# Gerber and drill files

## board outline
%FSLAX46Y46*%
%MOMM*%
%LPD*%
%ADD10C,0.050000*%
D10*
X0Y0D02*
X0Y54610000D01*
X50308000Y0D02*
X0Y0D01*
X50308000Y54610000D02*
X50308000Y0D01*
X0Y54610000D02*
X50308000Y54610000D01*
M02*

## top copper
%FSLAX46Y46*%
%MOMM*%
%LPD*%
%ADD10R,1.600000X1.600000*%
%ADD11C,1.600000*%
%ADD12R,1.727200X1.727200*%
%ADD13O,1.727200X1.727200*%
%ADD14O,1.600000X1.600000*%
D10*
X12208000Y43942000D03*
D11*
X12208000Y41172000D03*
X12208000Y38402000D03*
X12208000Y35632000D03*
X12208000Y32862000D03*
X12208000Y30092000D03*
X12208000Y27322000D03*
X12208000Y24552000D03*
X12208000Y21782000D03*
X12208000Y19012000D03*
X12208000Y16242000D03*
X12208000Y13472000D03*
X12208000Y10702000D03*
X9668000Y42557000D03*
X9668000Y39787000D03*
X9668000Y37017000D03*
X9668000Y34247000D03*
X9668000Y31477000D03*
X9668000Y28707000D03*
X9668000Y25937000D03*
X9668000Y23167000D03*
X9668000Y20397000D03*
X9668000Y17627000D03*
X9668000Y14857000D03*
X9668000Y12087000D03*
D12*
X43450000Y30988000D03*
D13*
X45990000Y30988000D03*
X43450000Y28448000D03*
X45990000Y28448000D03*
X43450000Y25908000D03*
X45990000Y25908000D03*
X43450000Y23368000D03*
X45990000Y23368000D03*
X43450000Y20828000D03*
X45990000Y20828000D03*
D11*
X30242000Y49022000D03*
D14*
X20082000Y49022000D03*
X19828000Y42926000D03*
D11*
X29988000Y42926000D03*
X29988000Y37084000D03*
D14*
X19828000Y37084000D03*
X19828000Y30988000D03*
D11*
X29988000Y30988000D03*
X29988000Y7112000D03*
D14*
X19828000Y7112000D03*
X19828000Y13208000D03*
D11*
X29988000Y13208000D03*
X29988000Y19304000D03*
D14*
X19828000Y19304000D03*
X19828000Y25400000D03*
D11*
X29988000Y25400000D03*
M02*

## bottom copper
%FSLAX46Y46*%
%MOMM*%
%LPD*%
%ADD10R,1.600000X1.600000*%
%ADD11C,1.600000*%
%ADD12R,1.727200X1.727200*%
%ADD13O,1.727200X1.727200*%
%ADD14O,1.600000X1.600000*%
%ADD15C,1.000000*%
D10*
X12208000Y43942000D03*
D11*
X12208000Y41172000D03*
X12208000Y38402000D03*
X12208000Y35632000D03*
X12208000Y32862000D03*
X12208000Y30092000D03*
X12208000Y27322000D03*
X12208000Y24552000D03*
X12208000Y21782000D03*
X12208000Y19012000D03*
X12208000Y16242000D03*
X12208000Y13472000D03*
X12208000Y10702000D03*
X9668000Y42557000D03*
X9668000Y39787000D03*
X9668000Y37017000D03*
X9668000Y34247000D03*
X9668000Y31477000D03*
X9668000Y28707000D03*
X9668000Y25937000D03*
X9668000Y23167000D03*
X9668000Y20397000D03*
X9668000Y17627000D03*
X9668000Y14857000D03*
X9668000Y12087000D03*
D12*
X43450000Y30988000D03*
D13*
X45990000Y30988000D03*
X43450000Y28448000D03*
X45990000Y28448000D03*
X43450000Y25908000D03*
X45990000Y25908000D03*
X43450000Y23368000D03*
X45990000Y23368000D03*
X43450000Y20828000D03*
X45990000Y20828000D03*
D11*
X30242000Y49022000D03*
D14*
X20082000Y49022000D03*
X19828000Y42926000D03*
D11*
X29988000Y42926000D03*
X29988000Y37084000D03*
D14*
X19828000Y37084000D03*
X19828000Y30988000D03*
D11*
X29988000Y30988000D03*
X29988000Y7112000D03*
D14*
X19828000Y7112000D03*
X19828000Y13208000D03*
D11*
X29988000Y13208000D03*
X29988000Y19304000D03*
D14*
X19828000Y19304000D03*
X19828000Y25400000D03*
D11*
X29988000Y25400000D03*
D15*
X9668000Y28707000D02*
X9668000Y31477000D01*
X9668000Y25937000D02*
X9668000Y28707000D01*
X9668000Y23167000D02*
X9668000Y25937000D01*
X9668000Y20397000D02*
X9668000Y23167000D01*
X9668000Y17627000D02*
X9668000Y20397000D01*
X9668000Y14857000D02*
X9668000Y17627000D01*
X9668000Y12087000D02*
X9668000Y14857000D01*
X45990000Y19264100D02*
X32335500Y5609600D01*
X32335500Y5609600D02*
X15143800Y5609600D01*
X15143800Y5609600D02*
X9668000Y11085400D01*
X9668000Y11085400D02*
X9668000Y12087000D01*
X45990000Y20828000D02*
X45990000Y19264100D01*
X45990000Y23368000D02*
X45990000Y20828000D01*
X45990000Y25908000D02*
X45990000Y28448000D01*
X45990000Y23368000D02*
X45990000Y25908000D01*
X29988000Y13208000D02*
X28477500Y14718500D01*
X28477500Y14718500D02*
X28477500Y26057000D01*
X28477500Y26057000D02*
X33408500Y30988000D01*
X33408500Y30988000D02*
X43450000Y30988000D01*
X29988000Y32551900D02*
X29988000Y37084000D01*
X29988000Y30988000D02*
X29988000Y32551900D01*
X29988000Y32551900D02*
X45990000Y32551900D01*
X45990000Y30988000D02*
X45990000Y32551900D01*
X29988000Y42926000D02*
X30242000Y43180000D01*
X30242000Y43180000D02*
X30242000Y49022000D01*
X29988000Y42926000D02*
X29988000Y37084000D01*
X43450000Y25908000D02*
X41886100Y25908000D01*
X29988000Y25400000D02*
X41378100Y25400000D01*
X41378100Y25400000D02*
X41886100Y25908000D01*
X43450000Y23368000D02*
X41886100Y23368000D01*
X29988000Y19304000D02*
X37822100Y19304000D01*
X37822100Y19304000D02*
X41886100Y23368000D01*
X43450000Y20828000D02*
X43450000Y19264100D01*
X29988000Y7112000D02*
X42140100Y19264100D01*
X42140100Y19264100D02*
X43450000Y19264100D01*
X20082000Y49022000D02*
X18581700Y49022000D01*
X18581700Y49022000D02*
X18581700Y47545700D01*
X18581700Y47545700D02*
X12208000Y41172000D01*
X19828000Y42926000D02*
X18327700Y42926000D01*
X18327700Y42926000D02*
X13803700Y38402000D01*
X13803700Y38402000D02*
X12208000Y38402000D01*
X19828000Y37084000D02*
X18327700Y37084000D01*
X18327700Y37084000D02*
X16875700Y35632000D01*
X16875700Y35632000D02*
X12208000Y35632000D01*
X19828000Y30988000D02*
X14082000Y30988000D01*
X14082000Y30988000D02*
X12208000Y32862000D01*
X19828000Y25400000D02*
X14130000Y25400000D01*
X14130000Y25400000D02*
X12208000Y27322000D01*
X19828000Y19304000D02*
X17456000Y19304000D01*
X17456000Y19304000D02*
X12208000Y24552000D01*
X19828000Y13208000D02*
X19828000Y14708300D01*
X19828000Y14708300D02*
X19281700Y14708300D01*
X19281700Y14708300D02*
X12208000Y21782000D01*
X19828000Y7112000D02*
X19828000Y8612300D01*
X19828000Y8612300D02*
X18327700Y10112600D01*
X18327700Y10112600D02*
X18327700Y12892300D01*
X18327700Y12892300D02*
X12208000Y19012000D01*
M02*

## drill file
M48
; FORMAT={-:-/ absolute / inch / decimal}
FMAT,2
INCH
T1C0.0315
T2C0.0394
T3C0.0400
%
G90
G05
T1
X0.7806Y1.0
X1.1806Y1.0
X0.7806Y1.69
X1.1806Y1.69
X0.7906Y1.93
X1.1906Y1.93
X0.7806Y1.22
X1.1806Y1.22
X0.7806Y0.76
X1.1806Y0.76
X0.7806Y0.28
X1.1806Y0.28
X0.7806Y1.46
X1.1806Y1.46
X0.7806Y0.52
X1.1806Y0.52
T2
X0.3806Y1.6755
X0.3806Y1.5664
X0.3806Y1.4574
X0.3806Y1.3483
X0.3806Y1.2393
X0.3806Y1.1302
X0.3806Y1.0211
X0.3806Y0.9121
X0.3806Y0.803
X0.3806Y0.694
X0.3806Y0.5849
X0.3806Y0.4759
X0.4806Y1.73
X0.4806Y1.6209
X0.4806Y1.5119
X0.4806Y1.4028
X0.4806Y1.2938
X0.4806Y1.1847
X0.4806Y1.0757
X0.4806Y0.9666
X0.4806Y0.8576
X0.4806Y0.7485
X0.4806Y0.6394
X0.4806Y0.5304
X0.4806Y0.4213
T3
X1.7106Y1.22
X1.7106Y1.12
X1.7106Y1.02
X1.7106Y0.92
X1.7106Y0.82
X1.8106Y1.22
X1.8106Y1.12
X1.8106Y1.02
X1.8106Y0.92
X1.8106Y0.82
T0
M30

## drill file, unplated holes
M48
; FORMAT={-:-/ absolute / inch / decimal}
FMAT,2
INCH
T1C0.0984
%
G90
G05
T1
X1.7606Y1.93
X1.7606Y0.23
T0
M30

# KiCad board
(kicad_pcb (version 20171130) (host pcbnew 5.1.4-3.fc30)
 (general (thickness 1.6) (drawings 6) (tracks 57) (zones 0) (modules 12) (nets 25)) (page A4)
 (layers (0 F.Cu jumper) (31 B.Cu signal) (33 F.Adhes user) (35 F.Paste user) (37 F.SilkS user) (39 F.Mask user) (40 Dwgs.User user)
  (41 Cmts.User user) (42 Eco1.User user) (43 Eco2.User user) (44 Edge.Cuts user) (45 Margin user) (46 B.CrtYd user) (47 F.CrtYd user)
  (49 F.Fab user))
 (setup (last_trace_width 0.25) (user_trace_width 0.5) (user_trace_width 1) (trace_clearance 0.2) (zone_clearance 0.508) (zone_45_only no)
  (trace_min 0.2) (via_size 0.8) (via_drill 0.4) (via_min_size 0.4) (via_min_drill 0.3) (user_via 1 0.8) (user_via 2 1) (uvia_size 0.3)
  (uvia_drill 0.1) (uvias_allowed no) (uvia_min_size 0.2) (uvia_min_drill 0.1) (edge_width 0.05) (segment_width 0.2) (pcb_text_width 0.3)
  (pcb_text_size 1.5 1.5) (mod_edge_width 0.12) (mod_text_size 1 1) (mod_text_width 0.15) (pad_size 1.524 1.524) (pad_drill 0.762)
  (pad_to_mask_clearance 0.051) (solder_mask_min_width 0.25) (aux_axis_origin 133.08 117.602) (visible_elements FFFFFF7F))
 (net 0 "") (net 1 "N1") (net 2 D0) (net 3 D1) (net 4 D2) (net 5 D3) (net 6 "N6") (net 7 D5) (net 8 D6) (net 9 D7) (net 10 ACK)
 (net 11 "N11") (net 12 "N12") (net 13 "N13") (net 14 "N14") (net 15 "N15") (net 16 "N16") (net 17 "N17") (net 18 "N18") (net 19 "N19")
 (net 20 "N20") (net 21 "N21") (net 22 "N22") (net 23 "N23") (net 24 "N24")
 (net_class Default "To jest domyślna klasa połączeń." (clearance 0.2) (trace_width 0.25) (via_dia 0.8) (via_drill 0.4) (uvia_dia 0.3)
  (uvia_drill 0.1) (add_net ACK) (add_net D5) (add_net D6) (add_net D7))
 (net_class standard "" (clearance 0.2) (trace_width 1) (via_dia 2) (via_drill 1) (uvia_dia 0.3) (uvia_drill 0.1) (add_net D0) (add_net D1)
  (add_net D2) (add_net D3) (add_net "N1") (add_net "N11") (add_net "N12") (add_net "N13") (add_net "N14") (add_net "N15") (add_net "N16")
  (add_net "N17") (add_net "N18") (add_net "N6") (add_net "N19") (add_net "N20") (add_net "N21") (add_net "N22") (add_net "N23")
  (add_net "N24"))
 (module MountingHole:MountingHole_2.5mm (layer F.Cu) (at 177.8 111.76)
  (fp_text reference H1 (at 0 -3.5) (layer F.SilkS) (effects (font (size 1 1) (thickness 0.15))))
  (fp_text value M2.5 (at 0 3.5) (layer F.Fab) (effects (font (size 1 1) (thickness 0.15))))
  (pad 1 np_thru_hole circle (at 0 0) (size 2.5 2.5) (drill 2.5) (layers *.Cu *.Mask)))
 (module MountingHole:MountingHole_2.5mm (layer F.Cu) (at 177.8 68.58)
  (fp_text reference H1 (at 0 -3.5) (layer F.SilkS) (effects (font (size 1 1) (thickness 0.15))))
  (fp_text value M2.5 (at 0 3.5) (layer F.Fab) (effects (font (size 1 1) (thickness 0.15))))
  (pad 1 np_thru_hole circle (at 0 0) (size 2.5 2.5) (drill 2.5) (layers *.Cu *.Mask)))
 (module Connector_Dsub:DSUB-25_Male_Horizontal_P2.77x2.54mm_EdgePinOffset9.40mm (layer F.Cu) (at 145.288 73.66 270)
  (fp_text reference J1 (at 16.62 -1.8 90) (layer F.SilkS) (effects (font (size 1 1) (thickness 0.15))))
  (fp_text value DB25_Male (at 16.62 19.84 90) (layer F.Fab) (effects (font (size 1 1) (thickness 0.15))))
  (pad 1 thru_hole rect (at 0 0 270) (size 1.6 1.6) (drill 1) (layers *.Cu *.Mask) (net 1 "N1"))
  (pad 2 thru_hole circle (at 2.77 0 270) (size 1.6 1.6) (drill 1) (layers *.Cu *.Mask) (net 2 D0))
  (pad 3 thru_hole circle (at 5.54 0 270) (size 1.6 1.6) (drill 1) (layers *.Cu *.Mask) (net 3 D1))
  (pad 4 thru_hole circle (at 8.31 0 270) (size 1.6 1.6) (drill 1) (layers *.Cu *.Mask) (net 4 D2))
  (pad 5 thru_hole circle (at 11.08 0 270) (size 1.6 1.6) (drill 1) (layers *.Cu *.Mask) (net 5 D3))
  (pad 6 thru_hole circle (at 13.85 0 270) (size 1.6 1.6) (drill 1) (layers *.Cu *.Mask) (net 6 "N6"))
  (pad 7 thru_hole circle (at 16.62 0 270) (size 1.6 1.6) (drill 1) (layers *.Cu *.Mask) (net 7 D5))
  (pad 8 thru_hole circle (at 19.39 0 270) (size 1.6 1.6) (drill 1) (layers *.Cu *.Mask) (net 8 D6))
  (pad 9 thru_hole circle (at 22.16 0 270) (size 1.6 1.6) (drill 1) (layers *.Cu *.Mask) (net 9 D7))
  (pad 10 thru_hole circle (at 24.93 0 270) (size 1.6 1.6) (drill 1) (layers *.Cu *.Mask) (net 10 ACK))
  (pad 11 thru_hole circle (at 27.7 0 270) (size 1.6 1.6) (drill 1) (layers *.Cu *.Mask) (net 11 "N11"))
  (pad 12 thru_hole circle (at 30.47 0 270) (size 1.6 1.6) (drill 1) (layers *.Cu *.Mask) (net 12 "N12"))
  (pad 13 thru_hole circle (at 33.24 0 270) (size 1.6 1.6) (drill 1) (layers *.Cu *.Mask) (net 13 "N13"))
  (pad 14 thru_hole circle (at 1.385 2.54 270) (size 1.6 1.6) (drill 1) (layers *.Cu *.Mask) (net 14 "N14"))
  (pad 15 thru_hole circle (at 4.155 2.54 270) (size 1.6 1.6) (drill 1) (layers *.Cu *.Mask) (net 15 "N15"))
  (pad 16 thru_hole circle (at 6.925 2.54 270) (size 1.6 1.6) (drill 1) (layers *.Cu *.Mask) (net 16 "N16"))
  (pad 17 thru_hole circle (at 9.695 2.54 270) (size 1.6 1.6) (drill 1) (layers *.Cu *.Mask) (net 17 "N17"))
  (pad 18 thru_hole circle (at 12.465 2.54 270) (size 1.6 1.6) (drill 1) (layers *.Cu *.Mask) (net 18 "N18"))
  (pad 19 thru_hole circle (at 15.235 2.54 270) (size 1.6 1.6) (drill 1) (layers *.Cu *.Mask) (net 18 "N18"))
  (pad 20 thru_hole circle (at 18.005 2.54 270) (size 1.6 1.6) (drill 1) (layers *.Cu *.Mask) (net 18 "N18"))
  (pad 21 thru_hole circle (at 20.775 2.54 270) (size 1.6 1.6) (drill 1) (layers *.Cu *.Mask) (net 18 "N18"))
  (pad 22 thru_hole circle (at 23.545 2.54 270) (size 1.6 1.6) (drill 1) (layers *.Cu *.Mask) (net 18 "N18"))
  (pad 23 thru_hole circle (at 26.315 2.54 270) (size 1.6 1.6) (drill 1) (layers *.Cu *.Mask) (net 18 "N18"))
  (pad 24 thru_hole circle (at 29.085 2.54 270) (size 1.6 1.6) (drill 1) (layers *.Cu *.Mask) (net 18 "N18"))
  (pad 25 thru_hole circle (at 31.855 2.54 270) (size 1.6 1.6) (drill 1) (layers *.Cu *.Mask) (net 18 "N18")))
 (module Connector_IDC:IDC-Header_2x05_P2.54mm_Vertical (layer F.Cu) (at 176.53 86.614)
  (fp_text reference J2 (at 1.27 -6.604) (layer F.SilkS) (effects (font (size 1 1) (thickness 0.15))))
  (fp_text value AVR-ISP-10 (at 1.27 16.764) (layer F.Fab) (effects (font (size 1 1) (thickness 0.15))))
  (pad 1 thru_hole rect (at 0 0) (size 1.7272 1.7272) (drill 1.016) (layers *.Cu *.Mask) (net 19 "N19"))
  (pad 2 thru_hole oval (at 2.54 0) (size 1.7272 1.7272) (drill 1.016) (layers *.Cu *.Mask) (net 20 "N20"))
  (pad 3 thru_hole oval (at 0 2.54) (size 1.7272 1.7272) (drill 1.016) (layers *.Cu *.Mask) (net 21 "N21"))
  (pad 4 thru_hole oval (at 2.54 2.54) (size 1.7272 1.7272) (drill 1.016) (layers *.Cu *.Mask) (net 18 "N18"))
  (pad 5 thru_hole oval (at 0 5.08) (size 1.7272 1.7272) (drill 1.016) (layers *.Cu *.Mask) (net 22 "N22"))
  (pad 6 thru_hole oval (at 2.54 5.08) (size 1.7272 1.7272) (drill 1.016) (layers *.Cu *.Mask) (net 18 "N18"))
  (pad 7 thru_hole oval (at 0 7.62) (size 1.7272 1.7272) (drill 1.016) (layers *.Cu *.Mask) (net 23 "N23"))
  (pad 8 thru_hole oval (at 2.54 7.62) (size 1.7272 1.7272) (drill 1.016) (layers *.Cu *.Mask) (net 18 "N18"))
  (pad 9 thru_hole oval (at 0 10.16) (size 1.7272 1.7272) (drill 1.016) (layers *.Cu *.Mask) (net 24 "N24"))
  (pad 10 thru_hole oval (at 2.54 10.16) (size 1.7272 1.7272) (drill 1.016) (layers *.Cu *.Mask) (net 18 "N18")))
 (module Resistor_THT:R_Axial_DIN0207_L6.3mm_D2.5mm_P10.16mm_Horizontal (layer F.Cu) (at 163.322 68.58 180)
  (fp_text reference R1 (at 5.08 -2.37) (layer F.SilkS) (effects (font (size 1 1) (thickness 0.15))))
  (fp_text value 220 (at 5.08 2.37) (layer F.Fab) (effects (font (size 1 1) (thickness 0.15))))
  (pad 1 thru_hole circle (at 0 0 180) (size 1.6 1.6) (drill 0.8) (layers *.Cu *.Mask) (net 20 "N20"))
  (pad 2 thru_hole oval (at 10.16 0 180) (size 1.6 1.6) (drill 0.8) (layers *.Cu *.Mask) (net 2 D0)))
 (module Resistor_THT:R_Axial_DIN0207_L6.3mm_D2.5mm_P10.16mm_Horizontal (layer F.Cu) (at 163.068 74.676 180)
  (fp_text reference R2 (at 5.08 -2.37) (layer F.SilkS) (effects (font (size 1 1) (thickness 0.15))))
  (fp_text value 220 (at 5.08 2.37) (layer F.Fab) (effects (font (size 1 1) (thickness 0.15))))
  (pad 2 thru_hole oval (at 10.16 0 180) (size 1.6 1.6) (drill 0.8) (layers *.Cu *.Mask) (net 3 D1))
  (pad 1 thru_hole circle (at 0 0 180) (size 1.6 1.6) (drill 0.8) (layers *.Cu *.Mask) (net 20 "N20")))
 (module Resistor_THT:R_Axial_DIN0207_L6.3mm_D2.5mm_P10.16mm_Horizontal (layer F.Cu) (at 163.068 80.518 180)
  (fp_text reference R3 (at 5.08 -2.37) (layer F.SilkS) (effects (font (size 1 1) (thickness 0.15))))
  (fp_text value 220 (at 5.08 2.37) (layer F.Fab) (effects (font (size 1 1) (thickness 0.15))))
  (pad 1 thru_hole circle (at 0 0 180) (size 1.6 1.6) (drill 0.8) (layers *.Cu *.Mask) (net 20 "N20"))
  (pad 2 thru_hole oval (at 10.16 0 180) (size 1.6 1.6) (drill 0.8) (layers *.Cu *.Mask) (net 4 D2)))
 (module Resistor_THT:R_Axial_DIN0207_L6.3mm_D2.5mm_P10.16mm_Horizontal (layer F.Cu) (at 163.068 86.614 180)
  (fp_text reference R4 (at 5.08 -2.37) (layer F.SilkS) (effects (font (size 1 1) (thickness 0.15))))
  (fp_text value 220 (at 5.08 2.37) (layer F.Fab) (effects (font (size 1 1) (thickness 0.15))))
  (pad 2 thru_hole oval (at 10.16 0 180) (size 1.6 1.6) (drill 0.8) (layers *.Cu *.Mask) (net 5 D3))
  (pad 1 thru_hole circle (at 0 0 180) (size 1.6 1.6) (drill 0.8) (layers *.Cu *.Mask) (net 20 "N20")))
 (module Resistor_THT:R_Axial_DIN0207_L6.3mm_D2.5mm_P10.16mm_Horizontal (layer F.Cu) (at 163.068 110.49 180)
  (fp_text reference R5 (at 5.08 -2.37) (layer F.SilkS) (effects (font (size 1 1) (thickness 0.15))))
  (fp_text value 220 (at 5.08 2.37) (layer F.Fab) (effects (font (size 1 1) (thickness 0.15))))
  (pad 1 thru_hole circle (at 0 0 180) (size 1.6 1.6) (drill 0.8) (layers *.Cu *.Mask) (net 24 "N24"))
  (pad 2 thru_hole oval (at 10.16 0 180) (size 1.6 1.6) (drill 0.8) (layers *.Cu *.Mask) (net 10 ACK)))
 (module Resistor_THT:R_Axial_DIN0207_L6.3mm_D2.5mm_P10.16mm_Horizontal (layer F.Cu) (at 163.068 104.394 180)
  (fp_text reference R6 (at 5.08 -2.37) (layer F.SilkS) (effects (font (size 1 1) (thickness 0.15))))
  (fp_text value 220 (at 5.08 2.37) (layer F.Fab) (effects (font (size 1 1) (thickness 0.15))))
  (pad 2 thru_hole oval (at 10.16 0 180) (size 1.6 1.6) (drill 0.8) (layers *.Cu *.Mask) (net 9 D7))
  (pad 1 thru_hole circle (at 0 0 180) (size 1.6 1.6) (drill 0.8) (layers *.Cu *.Mask) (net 19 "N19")))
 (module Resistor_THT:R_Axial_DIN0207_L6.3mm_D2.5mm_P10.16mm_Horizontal (layer F.Cu) (at 163.068 98.298 180)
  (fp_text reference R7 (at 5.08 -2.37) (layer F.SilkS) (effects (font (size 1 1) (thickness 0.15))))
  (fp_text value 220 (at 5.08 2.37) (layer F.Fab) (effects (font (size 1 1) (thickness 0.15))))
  (pad 1 thru_hole circle (at 0 0 180) (size 1.6 1.6) (drill 0.8) (layers *.Cu *.Mask) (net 23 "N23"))
  (pad 2 thru_hole oval (at 10.16 0 180) (size 1.6 1.6) (drill 0.8) (layers *.Cu *.Mask) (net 8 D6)))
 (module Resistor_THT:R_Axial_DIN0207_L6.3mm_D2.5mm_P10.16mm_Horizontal (layer F.Cu) (at 163.068 92.202 180)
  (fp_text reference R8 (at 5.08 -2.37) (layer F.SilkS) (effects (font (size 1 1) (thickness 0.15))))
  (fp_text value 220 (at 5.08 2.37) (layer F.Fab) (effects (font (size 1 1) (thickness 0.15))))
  (pad 2 thru_hole oval (at 10.16 0 180) (size 1.6 1.6) (drill 0.8) (layers *.Cu *.Mask) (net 7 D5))
  (pad 1 thru_hole circle (at 0 0 180) (size 1.6 1.6) (drill 0.8) (layers *.Cu *.Mask) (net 22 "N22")))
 (gr_line (start 133.08 117.602) (end 133.08 62.992) (layer Edge.Cuts) (width 0.05))
 (gr_line (start 183.388 117.602) (end 133.08 117.602) (layer Edge.Cuts) (width 0.05))
 (gr_line (start 183.388 62.992) (end 183.388 117.602) (layer Edge.Cuts) (width 0.05))
 (gr_line (start 133.08 62.992) (end 183.388 62.992) (layer Edge.Cuts) (width 0.05))
 (segment (start 142.748 88.895) (end 142.748 86.125) (width 1) (layer B.Cu) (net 18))
 (segment (start 142.748 91.665) (end 142.748 88.895) (width 1) (layer B.Cu) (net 18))
 (segment (start 142.748 94.435) (end 142.748 91.665) (width 1) (layer B.Cu) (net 18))
 (segment (start 142.748 97.205) (end 142.748 94.435) (width 1) (layer B.Cu) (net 18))
 (segment (start 142.748 99.975) (end 142.748 97.205) (width 1) (layer B.Cu) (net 18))
 (segment (start 142.748 102.745) (end 142.748 99.975) (width 1) (layer B.Cu) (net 18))
 (segment (start 142.748 105.515) (end 142.748 102.745) (width 1) (layer B.Cu) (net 18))
 (segment (start 179.07 98.3379) (end 165.4155 111.9924) (width 1) (layer B.Cu) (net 18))
 (segment (start 165.4155 111.9924) (end 148.2238 111.9924) (width 1) (layer B.Cu) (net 18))
 (segment (start 148.2238 111.9924) (end 142.748 106.5166) (width 1) (layer B.Cu) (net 18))
 (segment (start 142.748 106.5166) (end 142.748 105.515) (width 1) (layer B.Cu) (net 18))
 (segment (start 179.07 96.774) (end 179.07 98.3379) (width 1) (layer B.Cu) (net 18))
 (segment (start 179.07 94.234) (end 179.07 96.774) (width 1) (layer B.Cu) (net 18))
 (segment (start 179.07 91.694) (end 179.07 89.154) (width 1) (layer B.Cu) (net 18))
 (segment (start 179.07 94.234) (end 179.07 91.694) (width 1) (layer B.Cu) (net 18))
 (segment (start 163.068 104.394) (end 161.5575 102.8835) (width 1) (layer B.Cu) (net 19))
 (segment (start 161.5575 102.8835) (end 161.5575 91.545) (width 1) (layer B.Cu) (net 19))
 (segment (start 161.5575 91.545) (end 166.4885 86.614) (width 1) (layer B.Cu) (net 19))
 (segment (start 166.4885 86.614) (end 176.53 86.614) (width 1) (layer B.Cu) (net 19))
 (segment (start 163.068 85.0501) (end 163.068 80.518) (width 1) (layer B.Cu) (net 20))
 (segment (start 163.068 86.614) (end 163.068 85.0501) (width 1) (layer B.Cu) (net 20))
 (segment (start 163.068 85.0501) (end 179.07 85.0501) (width 1) (layer B.Cu) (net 20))
 (segment (start 179.07 86.614) (end 179.07 85.0501) (width 1) (layer B.Cu) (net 20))
 (segment (start 163.068 74.676) (end 163.322 74.422) (width 1) (layer B.Cu) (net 20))
 (segment (start 163.322 74.422) (end 163.322 68.58) (width 1) (layer B.Cu) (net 20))
 (segment (start 163.068 74.676) (end 163.068 80.518) (width 1) (layer B.Cu) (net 20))
 (segment (start 176.53 91.694) (end 174.9661 91.694) (width 1) (layer B.Cu) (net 22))
 (segment (start 163.068 92.202) (end 174.4581 92.202) (width 1) (layer B.Cu) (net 22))
 (segment (start 174.4581 92.202) (end 174.9661 91.694) (width 1) (layer B.Cu) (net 22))
 (segment (start 176.53 94.234) (end 174.9661 94.234) (width 1) (layer B.Cu) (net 23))
 (segment (start 163.068 98.298) (end 170.9021 98.298) (width 1) (layer B.Cu) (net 23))
 (segment (start 170.9021 98.298) (end 174.9661 94.234) (width 1) (layer B.Cu) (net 23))
 (segment (start 176.53 96.774) (end 176.53 98.3379) (width 1) (layer B.Cu) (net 24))
 (segment (start 163.068 110.49) (end 175.2201 98.3379) (width 1) (layer B.Cu) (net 24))
 (segment (start 175.2201 98.3379) (end 176.53 98.3379) (width 1) (layer B.Cu) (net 24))
 (segment (start 153.162 68.58) (end 151.6617 68.58) (width 1) (layer B.Cu) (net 2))
 (segment (start 151.6617 68.58) (end 151.6617 70.0563) (width 1) (layer B.Cu) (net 2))
 (segment (start 151.6617 70.0563) (end 145.288 76.43) (width 1) (layer B.Cu) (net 2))
 (segment (start 152.908 74.676) (end 151.4077 74.676) (width 1) (layer B.Cu) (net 3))
 (segment (start 151.4077 74.676) (end 146.8837 79.2) (width 1) (layer B.Cu) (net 3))
 (segment (start 146.8837 79.2) (end 145.288 79.2) (width 1) (layer B.Cu) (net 3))
 (segment (start 152.908 80.518) (end 151.4077 80.518) (width 1) (layer B.Cu) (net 4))
 (segment (start 151.4077 80.518) (end 149.9557 81.97) (width 1) (layer B.Cu) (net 4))
 (segment (start 149.9557 81.97) (end 145.288 81.97) (width 1) (layer B.Cu) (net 4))
 (segment (start 152.908 86.614) (end 147.162 86.614) (width 1) (layer B.Cu) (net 5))
 (segment (start 147.162 86.614) (end 145.288 84.74) (width 1) (layer B.Cu) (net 5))
 (segment (start 152.908 92.202) (end 147.21 92.202) (width 1) (layer B.Cu) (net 7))
 (segment (start 147.21 92.202) (end 145.288 90.28) (width 1) (layer B.Cu) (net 7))
 (segment (start 152.908 98.298) (end 150.536 98.298) (width 1) (layer B.Cu) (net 8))
 (segment (start 150.536 98.298) (end 145.288 93.05) (width 1) (layer B.Cu) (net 8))
 (segment (start 152.908 104.394) (end 152.908 102.8937) (width 1) (layer B.Cu) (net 9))
 (segment (start 152.908 102.8937) (end 152.3617 102.8937) (width 1) (layer B.Cu) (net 9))
 (segment (start 152.3617 102.8937) (end 145.288 95.82) (width 1) (layer B.Cu) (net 9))
 (segment (start 152.908 110.49) (end 152.908 108.9897) (width 1) (layer B.Cu) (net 10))
 (segment (start 152.908 108.9897) (end 151.4077 107.4894) (width 1) (layer B.Cu) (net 10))
 (segment (start 151.4077 107.4894) (end 151.4077 104.7097) (width 1) (layer B.Cu) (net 10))
 (segment (start 151.4077 104.7097) (end 145.288 98.59) (width 1) (layer B.Cu) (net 10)))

